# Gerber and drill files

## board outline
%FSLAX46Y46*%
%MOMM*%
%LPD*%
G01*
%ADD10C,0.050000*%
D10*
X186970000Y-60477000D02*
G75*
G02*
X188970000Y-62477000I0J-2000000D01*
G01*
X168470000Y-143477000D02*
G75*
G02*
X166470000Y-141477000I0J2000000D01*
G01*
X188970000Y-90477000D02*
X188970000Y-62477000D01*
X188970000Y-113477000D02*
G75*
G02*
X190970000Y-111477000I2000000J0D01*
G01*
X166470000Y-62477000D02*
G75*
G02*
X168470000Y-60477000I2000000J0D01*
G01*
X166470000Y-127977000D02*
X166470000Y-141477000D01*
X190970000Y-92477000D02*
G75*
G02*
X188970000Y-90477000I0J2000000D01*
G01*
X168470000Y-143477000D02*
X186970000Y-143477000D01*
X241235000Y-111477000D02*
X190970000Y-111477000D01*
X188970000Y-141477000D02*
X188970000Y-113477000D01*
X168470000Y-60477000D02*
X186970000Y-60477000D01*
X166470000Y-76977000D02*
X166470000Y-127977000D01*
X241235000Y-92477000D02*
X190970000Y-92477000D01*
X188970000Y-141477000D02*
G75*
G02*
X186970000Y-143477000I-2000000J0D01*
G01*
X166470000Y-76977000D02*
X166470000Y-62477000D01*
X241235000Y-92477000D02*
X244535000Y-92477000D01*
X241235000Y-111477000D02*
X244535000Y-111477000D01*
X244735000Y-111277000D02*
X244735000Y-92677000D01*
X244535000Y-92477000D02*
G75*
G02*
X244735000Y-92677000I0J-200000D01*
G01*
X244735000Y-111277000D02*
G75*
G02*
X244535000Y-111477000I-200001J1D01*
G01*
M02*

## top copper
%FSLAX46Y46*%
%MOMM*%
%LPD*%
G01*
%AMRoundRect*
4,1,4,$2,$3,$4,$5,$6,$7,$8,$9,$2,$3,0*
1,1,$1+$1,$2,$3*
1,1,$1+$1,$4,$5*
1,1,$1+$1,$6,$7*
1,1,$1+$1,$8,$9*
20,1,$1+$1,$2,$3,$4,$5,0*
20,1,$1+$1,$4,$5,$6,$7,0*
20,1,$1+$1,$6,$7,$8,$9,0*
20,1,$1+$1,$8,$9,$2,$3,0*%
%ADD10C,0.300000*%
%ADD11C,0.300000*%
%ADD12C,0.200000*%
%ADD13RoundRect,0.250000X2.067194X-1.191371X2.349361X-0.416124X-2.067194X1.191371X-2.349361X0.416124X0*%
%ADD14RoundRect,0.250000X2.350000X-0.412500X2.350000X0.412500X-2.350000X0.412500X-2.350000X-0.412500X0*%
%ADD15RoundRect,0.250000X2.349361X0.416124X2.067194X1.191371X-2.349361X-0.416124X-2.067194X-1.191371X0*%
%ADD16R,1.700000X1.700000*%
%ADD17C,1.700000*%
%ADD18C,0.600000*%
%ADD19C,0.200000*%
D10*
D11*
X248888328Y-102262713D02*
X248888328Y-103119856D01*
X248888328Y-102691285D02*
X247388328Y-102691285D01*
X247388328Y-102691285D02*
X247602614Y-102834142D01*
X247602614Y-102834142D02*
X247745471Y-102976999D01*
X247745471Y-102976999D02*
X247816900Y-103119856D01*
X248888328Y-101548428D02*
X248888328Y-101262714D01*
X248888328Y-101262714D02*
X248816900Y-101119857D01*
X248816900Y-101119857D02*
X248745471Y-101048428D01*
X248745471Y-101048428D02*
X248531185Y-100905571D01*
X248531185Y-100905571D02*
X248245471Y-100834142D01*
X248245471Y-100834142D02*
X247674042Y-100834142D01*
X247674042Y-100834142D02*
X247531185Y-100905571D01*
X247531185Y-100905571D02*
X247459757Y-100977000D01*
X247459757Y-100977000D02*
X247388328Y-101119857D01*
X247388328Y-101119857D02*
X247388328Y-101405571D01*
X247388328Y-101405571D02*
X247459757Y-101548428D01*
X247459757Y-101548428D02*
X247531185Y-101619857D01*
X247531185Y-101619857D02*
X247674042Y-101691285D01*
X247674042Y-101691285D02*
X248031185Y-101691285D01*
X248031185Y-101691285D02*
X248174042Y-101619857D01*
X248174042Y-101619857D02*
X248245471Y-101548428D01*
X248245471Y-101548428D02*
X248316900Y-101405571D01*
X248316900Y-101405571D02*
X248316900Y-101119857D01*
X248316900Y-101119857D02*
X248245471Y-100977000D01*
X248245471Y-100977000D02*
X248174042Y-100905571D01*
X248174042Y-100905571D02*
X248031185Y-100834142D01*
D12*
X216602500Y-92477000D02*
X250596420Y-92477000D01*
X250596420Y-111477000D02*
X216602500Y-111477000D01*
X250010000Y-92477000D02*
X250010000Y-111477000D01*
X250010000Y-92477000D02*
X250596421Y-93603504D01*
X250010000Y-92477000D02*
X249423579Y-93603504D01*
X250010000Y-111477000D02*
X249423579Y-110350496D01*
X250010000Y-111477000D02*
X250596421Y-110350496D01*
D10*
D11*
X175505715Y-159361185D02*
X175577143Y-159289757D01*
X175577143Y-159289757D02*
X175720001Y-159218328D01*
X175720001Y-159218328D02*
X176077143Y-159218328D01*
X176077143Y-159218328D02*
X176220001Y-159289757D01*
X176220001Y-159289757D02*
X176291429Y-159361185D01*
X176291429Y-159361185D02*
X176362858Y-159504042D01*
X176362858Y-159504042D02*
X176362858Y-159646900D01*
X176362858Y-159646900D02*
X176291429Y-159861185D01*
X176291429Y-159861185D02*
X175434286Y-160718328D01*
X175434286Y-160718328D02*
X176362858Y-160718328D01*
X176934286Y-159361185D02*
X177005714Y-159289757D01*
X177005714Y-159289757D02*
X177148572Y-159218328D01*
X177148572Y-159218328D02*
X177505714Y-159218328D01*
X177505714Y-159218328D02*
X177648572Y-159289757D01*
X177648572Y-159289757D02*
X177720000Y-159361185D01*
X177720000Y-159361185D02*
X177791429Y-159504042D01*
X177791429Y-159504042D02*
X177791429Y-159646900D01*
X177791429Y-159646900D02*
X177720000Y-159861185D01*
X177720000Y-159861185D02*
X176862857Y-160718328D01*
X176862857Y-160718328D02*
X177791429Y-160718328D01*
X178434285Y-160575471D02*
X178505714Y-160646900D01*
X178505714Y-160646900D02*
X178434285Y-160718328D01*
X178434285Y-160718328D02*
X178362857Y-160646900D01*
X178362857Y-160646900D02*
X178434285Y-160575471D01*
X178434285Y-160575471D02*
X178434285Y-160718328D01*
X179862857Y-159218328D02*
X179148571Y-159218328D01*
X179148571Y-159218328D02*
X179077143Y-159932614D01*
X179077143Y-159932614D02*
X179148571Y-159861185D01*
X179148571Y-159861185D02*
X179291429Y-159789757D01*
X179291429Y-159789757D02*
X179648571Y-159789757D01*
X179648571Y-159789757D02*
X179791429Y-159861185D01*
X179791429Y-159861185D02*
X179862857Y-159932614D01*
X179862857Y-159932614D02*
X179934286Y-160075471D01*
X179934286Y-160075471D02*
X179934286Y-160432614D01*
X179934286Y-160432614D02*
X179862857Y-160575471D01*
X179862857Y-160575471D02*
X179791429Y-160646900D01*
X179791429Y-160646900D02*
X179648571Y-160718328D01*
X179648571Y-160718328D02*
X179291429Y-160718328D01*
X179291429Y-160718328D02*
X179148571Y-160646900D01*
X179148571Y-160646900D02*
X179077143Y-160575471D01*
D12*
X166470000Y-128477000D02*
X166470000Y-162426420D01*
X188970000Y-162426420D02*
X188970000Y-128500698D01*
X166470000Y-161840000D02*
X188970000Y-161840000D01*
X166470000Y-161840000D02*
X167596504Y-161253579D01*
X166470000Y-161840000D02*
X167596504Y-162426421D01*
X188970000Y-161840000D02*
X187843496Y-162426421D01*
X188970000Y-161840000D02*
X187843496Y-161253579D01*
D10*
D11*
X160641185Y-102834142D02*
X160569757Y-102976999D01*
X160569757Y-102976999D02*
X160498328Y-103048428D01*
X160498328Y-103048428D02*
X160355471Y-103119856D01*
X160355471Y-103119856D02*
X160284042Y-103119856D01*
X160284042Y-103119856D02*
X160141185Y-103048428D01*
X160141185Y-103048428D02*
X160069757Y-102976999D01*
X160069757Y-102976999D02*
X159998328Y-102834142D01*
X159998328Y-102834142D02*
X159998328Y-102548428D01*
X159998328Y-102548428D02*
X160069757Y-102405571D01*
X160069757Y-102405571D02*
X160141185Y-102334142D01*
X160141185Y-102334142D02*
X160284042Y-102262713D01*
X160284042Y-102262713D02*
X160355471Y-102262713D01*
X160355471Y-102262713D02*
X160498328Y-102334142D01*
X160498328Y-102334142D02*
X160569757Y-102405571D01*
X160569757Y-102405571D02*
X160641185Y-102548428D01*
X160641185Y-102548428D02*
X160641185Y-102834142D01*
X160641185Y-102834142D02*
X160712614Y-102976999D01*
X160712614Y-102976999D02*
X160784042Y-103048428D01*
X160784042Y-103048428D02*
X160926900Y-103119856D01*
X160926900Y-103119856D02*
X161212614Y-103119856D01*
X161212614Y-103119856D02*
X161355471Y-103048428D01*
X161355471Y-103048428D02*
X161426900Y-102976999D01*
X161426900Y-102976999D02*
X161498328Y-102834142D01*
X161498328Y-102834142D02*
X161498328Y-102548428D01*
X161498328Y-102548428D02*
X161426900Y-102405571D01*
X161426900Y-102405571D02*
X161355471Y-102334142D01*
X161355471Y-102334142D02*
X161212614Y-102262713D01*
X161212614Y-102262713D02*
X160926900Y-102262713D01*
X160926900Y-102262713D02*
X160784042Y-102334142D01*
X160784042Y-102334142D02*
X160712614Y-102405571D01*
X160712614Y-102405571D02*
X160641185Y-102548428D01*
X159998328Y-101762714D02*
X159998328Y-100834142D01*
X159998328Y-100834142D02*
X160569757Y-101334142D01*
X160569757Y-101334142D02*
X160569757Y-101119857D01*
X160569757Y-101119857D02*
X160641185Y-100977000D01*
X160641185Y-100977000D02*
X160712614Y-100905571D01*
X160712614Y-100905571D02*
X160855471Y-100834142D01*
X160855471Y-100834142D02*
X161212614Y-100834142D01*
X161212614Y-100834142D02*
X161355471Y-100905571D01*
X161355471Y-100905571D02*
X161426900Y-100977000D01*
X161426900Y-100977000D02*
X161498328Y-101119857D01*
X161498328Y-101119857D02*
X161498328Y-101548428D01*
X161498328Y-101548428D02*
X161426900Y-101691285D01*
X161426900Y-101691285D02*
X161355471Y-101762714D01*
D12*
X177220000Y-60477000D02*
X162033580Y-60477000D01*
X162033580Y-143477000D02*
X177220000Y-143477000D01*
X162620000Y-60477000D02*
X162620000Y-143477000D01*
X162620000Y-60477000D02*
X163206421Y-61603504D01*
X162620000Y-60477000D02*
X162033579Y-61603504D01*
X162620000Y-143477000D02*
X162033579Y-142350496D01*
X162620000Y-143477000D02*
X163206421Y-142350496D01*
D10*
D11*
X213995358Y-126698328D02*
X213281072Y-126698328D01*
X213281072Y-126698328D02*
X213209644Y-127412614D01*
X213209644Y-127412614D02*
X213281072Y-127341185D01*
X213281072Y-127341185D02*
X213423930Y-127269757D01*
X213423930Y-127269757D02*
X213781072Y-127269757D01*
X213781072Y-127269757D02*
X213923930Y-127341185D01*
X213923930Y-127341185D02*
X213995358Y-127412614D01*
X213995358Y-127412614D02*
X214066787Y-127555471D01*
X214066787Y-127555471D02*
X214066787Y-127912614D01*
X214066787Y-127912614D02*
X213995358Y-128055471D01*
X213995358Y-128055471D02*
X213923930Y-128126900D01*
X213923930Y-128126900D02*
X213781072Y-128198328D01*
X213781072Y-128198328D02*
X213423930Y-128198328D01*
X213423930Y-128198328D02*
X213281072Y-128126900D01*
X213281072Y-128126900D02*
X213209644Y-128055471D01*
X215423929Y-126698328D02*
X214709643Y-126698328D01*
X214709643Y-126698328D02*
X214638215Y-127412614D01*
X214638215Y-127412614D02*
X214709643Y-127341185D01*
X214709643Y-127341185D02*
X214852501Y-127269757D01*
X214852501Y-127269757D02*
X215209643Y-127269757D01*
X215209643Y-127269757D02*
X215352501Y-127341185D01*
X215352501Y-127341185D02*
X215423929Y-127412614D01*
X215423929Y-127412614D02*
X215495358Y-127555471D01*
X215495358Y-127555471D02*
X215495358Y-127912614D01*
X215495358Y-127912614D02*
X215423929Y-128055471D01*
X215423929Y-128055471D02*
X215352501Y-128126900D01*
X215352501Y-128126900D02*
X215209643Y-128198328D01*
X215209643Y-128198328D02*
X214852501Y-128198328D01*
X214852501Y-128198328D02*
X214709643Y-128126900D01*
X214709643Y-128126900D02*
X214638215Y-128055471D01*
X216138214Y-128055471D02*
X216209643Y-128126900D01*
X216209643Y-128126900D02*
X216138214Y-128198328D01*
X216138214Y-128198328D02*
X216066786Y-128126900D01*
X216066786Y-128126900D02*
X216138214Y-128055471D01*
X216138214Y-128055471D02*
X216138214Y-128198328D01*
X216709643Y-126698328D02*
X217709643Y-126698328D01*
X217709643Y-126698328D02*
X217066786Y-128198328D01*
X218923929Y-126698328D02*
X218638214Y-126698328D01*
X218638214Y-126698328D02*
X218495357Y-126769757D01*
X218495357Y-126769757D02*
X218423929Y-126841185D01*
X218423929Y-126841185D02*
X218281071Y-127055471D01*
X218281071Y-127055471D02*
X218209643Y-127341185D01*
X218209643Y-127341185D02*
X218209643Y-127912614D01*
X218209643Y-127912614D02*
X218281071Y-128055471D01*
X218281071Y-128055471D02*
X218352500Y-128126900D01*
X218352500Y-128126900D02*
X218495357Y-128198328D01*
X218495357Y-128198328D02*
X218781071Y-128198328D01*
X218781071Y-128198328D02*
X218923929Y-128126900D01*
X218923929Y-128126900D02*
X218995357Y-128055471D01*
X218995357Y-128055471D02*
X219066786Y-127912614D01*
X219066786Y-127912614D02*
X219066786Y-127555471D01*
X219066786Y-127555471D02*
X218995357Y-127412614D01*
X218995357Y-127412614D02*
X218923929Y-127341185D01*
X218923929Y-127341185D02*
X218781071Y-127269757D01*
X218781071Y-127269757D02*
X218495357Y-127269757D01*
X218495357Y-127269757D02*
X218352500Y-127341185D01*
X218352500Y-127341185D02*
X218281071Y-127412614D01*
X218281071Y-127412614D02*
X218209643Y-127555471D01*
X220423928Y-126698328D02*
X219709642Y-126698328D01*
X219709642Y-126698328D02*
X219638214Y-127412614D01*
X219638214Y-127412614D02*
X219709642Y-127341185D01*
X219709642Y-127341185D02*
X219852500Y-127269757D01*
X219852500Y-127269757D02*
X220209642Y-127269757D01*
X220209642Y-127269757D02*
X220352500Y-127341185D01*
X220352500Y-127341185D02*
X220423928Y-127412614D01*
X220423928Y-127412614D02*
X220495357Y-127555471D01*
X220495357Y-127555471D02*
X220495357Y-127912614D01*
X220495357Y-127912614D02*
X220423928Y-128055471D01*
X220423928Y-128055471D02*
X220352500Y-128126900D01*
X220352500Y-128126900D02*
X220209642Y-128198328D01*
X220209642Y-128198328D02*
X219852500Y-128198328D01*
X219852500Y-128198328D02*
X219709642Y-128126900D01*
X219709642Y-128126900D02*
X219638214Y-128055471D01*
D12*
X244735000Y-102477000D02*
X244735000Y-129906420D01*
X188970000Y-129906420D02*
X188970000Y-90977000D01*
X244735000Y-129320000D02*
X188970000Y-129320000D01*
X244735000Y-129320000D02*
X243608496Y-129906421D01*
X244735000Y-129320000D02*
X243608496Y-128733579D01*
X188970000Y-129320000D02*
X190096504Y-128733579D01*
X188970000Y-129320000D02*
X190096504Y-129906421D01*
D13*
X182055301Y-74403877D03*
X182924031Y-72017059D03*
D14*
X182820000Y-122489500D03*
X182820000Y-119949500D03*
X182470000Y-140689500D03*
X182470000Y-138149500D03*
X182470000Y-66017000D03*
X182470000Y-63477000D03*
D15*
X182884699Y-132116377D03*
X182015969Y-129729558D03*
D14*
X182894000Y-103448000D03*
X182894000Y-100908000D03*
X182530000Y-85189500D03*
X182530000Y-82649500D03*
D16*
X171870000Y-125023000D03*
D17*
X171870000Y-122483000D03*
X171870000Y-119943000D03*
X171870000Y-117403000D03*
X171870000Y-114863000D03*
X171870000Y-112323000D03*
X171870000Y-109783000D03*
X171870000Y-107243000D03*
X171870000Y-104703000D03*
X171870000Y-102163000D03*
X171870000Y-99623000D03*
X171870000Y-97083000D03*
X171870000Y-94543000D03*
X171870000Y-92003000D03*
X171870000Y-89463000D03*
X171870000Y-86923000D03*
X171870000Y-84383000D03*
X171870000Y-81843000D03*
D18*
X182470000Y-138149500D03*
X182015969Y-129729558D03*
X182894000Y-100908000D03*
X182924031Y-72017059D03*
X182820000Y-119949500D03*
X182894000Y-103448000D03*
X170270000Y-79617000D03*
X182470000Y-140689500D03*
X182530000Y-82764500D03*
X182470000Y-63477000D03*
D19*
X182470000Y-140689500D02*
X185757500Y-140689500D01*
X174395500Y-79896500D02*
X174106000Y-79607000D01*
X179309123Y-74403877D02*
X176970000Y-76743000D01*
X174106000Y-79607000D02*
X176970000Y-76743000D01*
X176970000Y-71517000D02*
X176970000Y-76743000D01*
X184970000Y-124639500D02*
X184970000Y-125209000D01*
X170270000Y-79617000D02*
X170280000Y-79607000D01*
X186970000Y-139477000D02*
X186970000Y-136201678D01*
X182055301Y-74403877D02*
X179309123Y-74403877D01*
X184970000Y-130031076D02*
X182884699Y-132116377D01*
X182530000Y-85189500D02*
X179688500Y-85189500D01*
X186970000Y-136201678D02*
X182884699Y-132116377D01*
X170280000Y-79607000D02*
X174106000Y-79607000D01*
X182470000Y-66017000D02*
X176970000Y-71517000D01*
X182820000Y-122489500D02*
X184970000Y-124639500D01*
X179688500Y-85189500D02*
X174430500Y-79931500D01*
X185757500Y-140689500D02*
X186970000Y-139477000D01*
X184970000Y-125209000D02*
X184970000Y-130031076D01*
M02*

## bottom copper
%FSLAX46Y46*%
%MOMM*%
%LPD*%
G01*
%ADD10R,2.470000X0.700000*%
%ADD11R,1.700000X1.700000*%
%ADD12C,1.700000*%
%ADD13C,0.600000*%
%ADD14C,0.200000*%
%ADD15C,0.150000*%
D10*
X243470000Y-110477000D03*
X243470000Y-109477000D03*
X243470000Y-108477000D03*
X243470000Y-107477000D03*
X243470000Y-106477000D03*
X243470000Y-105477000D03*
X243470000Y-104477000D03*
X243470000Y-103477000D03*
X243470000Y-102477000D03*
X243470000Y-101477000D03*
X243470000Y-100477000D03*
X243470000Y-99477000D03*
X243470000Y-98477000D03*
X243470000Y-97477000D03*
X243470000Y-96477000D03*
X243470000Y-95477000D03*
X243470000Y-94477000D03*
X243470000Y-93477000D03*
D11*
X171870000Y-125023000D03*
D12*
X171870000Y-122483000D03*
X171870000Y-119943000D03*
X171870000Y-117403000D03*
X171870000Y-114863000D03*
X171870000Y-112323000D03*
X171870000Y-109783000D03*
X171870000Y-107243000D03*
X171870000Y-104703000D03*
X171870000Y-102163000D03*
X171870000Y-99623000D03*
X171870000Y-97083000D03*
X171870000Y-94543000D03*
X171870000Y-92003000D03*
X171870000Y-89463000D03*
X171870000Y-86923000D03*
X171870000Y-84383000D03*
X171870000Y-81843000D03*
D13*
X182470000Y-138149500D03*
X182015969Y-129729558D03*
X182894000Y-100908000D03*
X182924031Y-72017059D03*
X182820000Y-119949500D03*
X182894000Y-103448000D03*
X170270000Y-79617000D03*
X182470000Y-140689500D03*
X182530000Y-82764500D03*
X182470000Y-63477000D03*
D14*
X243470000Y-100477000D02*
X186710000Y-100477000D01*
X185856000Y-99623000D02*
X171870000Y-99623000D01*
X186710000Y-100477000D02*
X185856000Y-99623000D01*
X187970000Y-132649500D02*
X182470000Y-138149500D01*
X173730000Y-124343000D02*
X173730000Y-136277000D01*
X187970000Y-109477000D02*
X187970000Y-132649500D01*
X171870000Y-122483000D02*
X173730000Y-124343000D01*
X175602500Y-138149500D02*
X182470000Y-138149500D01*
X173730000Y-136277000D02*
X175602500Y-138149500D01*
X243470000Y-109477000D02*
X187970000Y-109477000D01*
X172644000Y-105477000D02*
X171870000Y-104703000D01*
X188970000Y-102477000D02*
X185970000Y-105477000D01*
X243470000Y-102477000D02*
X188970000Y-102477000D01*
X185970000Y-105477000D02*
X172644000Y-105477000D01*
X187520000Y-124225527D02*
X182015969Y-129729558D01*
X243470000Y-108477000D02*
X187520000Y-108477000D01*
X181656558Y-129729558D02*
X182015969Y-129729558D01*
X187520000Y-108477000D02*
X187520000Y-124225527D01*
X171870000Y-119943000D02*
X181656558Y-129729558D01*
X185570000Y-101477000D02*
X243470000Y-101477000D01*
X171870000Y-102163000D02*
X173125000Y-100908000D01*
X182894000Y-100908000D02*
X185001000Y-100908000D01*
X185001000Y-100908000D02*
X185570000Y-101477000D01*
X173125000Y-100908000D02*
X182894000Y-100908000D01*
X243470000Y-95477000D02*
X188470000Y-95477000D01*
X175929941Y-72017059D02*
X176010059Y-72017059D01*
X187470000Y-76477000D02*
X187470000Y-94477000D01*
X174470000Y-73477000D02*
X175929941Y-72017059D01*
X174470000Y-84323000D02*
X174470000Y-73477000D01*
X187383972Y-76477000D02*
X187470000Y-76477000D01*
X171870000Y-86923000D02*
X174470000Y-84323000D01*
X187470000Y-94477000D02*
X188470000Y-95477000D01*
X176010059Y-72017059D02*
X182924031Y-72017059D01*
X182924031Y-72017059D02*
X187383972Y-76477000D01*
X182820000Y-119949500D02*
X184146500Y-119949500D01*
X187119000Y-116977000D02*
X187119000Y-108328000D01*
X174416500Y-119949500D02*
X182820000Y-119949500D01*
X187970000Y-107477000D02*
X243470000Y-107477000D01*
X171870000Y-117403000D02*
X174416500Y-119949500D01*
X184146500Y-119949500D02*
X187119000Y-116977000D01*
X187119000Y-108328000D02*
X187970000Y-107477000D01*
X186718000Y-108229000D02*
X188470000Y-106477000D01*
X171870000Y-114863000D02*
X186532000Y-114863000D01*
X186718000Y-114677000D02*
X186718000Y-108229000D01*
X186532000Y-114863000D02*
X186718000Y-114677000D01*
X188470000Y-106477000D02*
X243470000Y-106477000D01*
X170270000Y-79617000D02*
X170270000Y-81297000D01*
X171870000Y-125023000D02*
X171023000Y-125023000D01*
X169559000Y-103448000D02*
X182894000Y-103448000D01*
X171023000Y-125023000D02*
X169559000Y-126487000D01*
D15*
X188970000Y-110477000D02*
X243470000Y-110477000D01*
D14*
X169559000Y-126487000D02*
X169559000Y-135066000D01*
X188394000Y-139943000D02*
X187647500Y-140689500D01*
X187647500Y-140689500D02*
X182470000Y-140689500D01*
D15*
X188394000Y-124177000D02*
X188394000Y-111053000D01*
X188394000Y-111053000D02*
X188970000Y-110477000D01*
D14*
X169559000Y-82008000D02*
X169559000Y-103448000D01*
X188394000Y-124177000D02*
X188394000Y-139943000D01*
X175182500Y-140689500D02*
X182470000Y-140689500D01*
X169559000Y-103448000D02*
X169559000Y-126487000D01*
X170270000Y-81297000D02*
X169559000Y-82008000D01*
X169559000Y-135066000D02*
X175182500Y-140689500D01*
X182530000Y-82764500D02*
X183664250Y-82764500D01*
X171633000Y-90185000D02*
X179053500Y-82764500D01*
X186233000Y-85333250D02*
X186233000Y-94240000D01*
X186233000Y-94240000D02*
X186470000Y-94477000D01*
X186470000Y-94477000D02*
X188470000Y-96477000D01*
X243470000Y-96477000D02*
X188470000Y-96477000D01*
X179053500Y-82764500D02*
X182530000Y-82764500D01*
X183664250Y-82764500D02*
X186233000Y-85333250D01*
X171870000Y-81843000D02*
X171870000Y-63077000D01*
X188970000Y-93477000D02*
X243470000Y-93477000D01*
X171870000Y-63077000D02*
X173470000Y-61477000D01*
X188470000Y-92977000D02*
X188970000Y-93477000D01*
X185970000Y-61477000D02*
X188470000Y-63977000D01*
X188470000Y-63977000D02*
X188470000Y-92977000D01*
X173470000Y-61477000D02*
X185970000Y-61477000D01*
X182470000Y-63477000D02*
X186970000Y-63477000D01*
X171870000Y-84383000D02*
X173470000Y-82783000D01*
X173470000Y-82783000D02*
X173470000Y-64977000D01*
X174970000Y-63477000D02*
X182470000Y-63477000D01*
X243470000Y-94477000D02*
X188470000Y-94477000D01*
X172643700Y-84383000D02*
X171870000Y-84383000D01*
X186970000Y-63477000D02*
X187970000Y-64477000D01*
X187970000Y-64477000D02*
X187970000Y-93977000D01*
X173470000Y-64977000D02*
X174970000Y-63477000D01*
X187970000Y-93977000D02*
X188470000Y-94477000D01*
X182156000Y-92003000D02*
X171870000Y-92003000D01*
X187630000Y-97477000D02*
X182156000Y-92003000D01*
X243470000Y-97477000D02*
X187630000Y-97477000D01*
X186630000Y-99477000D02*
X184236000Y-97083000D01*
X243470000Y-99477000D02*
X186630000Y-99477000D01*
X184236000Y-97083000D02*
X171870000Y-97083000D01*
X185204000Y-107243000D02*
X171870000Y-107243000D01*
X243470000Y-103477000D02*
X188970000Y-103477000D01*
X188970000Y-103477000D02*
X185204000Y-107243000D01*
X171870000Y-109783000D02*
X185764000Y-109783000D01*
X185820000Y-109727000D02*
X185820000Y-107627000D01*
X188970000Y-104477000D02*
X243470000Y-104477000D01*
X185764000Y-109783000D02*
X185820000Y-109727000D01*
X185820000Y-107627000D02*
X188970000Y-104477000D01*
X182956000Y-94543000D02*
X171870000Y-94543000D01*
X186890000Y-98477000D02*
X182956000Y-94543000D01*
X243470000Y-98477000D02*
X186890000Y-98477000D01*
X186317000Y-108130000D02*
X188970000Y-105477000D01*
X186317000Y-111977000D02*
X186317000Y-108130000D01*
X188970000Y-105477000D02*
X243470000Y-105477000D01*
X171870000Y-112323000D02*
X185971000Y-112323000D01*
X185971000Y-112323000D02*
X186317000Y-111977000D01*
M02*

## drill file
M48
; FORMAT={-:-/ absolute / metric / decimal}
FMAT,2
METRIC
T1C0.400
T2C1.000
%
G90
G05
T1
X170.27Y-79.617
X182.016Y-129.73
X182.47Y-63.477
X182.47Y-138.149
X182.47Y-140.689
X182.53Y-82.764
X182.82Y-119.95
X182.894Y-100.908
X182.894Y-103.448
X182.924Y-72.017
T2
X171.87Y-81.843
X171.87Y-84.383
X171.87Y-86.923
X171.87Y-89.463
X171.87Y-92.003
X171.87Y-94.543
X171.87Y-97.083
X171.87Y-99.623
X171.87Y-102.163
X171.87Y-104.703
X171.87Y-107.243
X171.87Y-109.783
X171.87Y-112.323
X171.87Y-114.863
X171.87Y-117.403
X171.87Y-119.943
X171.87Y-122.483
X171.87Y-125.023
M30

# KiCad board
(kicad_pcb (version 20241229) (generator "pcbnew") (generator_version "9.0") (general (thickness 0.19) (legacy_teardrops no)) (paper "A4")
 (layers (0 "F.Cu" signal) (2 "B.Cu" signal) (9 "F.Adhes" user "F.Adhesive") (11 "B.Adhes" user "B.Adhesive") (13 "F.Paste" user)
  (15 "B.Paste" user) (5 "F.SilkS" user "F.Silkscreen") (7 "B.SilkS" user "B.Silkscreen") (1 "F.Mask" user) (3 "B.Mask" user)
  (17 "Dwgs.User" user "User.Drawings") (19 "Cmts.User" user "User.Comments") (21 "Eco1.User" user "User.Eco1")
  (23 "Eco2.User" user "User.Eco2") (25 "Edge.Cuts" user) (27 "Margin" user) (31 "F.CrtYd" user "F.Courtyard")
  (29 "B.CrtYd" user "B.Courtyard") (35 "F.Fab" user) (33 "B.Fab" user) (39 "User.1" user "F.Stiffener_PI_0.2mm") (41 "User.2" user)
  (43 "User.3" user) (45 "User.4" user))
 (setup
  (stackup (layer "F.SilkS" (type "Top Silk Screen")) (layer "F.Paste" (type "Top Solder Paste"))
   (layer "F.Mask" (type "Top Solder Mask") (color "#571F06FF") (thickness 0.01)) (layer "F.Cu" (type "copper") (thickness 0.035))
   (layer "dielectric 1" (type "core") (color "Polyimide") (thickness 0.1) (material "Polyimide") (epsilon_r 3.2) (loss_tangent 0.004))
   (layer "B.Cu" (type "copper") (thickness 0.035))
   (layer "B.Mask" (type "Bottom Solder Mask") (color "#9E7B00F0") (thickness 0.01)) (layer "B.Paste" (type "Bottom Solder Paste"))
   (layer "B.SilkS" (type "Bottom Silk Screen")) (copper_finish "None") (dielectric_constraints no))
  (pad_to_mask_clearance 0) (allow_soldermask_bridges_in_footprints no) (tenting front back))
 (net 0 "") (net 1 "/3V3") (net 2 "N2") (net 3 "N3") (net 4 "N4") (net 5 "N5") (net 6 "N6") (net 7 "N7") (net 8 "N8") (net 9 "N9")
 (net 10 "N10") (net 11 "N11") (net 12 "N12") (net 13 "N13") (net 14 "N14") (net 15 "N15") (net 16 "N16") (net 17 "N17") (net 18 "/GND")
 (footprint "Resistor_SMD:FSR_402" (layer "F.Cu") (at 182.47 73.2645 70)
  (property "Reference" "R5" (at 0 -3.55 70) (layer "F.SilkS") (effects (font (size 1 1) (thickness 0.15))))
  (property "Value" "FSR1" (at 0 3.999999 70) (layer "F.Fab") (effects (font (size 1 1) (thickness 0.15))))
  (pad "1" smd roundrect (at -1.2125 0 70) (size 1.325 5.2) (layers "F.Cu" "F.Mask" "F.Paste") (roundrect_rratio 0.188679) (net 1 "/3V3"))
  (pad "2" smd roundrect (at 1.327499 0 70) (size 1.325 5.2) (layers "F.Cu" "F.Mask" "F.Paste") (roundrect_rratio 0.188679) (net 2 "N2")))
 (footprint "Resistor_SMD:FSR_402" (layer "F.Cu") (at 182.82 121.277 90)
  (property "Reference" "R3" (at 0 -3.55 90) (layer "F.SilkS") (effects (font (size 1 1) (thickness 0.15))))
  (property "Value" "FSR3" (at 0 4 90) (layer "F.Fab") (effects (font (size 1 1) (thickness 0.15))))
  (pad "1" smd roundrect (at -1.2125 0 90) (size 1.325 5.2) (layers "F.Cu" "F.Mask" "F.Paste") (roundrect_rratio 0.188679) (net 1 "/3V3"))
  (pad "2" smd roundrect (at 1.3275 0 90) (size 1.325 5.2) (layers "F.Cu" "F.Mask" "F.Paste") (roundrect_rratio 0.188679) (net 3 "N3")))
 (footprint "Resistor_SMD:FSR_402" (layer "F.Cu") (at 182.47 139.477 90)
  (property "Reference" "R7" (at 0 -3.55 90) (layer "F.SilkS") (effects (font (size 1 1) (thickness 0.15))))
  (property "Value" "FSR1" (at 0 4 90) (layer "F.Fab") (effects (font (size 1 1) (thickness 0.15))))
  (pad "1" smd roundrect (at -1.2125 0 90) (size 1.325 5.2) (layers "F.Cu" "F.Mask" "F.Paste") (roundrect_rratio 0.188679) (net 1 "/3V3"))
  (pad "2" smd roundrect (at 1.3275 0 90) (size 1.325 5.2) (layers "F.Cu" "F.Mask" "F.Paste") (roundrect_rratio 0.188679) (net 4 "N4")))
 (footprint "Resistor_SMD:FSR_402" (layer "F.Cu") (at 182.47 64.8045 90)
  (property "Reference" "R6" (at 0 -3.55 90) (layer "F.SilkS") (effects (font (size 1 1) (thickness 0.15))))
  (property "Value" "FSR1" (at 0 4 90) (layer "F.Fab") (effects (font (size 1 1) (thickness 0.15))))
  (pad "1" smd roundrect (at -1.2125 0 90) (size 1.325 5.2) (layers "F.Cu" "F.Mask" "F.Paste") (roundrect_rratio 0.188679) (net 1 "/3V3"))
  (pad "2" smd roundrect (at 1.3275 0 90) (size 1.325 5.2) (layers "F.Cu" "F.Mask" "F.Paste") (roundrect_rratio 0.188679) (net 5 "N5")))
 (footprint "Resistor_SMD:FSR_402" (layer "F.Cu") (at 182.47 130.977 110)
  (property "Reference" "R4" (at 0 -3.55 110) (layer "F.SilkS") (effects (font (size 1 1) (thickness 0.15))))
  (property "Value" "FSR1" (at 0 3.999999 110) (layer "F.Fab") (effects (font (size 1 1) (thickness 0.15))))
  (pad "1" smd roundrect (at -1.2125 0 110) (size 1.325 5.2) (layers "F.Cu" "F.Mask" "F.Paste") (roundrect_rratio 0.188679) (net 1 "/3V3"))
  (pad "2" smd roundrect (at 1.3275 0.000001 110) (size 1.325 5.2) (layers "F.Cu" "F.Mask" "F.Paste") (roundrect_rratio 0.188679)
   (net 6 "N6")))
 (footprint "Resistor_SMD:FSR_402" (layer "F.Cu") (at 182.894 102.2355 90)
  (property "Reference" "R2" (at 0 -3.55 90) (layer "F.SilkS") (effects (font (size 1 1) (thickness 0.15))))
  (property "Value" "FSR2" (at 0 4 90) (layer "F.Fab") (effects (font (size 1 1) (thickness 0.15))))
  (pad "1" smd roundrect (at -1.2125 0 90) (size 1.325 5.2) (layers "F.Cu" "F.Mask" "F.Paste") (roundrect_rratio 0.188679) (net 1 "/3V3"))
  (pad "2" smd roundrect (at 1.3275 0 90) (size 1.325 5.2) (layers "F.Cu" "F.Mask" "F.Paste") (roundrect_rratio 0.188679) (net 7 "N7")))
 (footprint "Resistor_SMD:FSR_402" (layer "F.Cu") (at 182.53 83.977 90)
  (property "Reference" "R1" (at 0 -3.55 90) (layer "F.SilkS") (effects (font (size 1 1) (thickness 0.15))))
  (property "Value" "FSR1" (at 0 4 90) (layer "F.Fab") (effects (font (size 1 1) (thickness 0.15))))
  (pad "1" smd roundrect (at -1.2125 0 90) (size 1.325 5.2) (layers "F.Cu" "F.Mask" "F.Paste") (roundrect_rratio 0.188679) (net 1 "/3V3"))
  (pad "2" smd roundrect (at 1.3275 0 90) (size 1.325 5.2) (layers "F.Cu" "F.Mask" "F.Paste") (roundrect_rratio 0.188679) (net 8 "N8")))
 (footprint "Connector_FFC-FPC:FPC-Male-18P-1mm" (layer "B.Cu") (at 243.43 102.387 90)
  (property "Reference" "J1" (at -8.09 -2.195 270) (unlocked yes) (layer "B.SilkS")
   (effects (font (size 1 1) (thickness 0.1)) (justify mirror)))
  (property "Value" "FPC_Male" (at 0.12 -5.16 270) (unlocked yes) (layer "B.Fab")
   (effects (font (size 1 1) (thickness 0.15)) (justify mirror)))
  (fp_line (start 9.91 -2.195) (end 9.91 1.105) (stroke (width 0.05) (type default)) (layer "Edge.Cuts"))
  (fp_line (start -9.09 -2.195) (end -9.09 1.105) (stroke (width 0.05) (type default)) (layer "Edge.Cuts"))
  (fp_line (start -8.89 1.305) (end 9.71 1.305) (stroke (width 0.05) (type default)) (layer "Edge.Cuts"))
  (fp_arc (start 9.91 1.105) (mid 9.851421 1.246421) (end 9.71 1.305) (stroke (width 0.05) (type default)) (layer "Edge.Cuts"))
  (fp_arc (start -8.89 1.305) (mid -9.031421 1.246421) (end -9.09 1.105) (stroke (width 0.05) (type default)) (layer "Edge.Cuts"))
  (pad "1" smd rect (at -8.09 0.04) (size 2.47 0.7) (layers "B.Cu" "B.Mask" "B.Paste") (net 1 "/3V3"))
  (pad "2" smd rect (at -7.09 0.04) (size 2.47 0.7) (layers "B.Cu" "B.Mask" "B.Paste") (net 4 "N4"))
  (pad "3" smd rect (at -6.09 0.04) (size 2.47 0.7) (layers "B.Cu" "B.Mask" "B.Paste") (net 6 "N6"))
  (pad "4" smd rect (at -5.09 0.04) (size 2.47 0.7) (layers "B.Cu" "B.Mask" "B.Paste") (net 3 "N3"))
  (pad "5" smd rect (at -4.09 0.04) (size 2.47 0.7) (layers "B.Cu" "B.Mask" "B.Paste") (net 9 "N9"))
  (pad "6" smd rect (at -3.09 0.04) (size 2.47 0.7) (layers "B.Cu" "B.Mask" "B.Paste") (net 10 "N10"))
  (pad "7" smd rect (at -2.09 0.04) (size 2.47 0.7) (layers "B.Cu" "B.Mask" "B.Paste") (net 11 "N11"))
  (pad "8" smd rect (at -1.09 0.04) (size 2.47 0.7) (layers "B.Cu" "B.Mask" "B.Paste") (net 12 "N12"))
  (pad "9" smd rect (at -0.09 0.04) (size 2.47 0.7) (layers "B.Cu" "B.Mask" "B.Paste") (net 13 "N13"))
  (pad "10" smd rect (at 0.91 0.04) (size 2.47 0.7) (layers "B.Cu" "B.Mask" "B.Paste") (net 7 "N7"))
  (pad "11" smd rect (at 1.91 0.04) (size 2.47 0.7) (layers "B.Cu" "B.Mask" "B.Paste") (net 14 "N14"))
  (pad "12" smd rect (at 2.91 0.04) (size 2.47 0.7) (layers "B.Cu" "B.Mask" "B.Paste") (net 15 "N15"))
  (pad "13" smd rect (at 3.91 0.04) (size 2.47 0.7) (layers "B.Cu" "B.Mask" "B.Paste") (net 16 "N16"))
  (pad "14" smd rect (at 4.91 0.04) (size 2.47 0.7) (layers "B.Cu" "B.Mask" "B.Paste") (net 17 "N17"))
  (pad "15" smd rect (at 5.91 0.04) (size 2.47 0.7) (layers "B.Cu" "B.Mask" "B.Paste") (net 8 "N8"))
  (pad "16" smd rect (at 6.91 0.04) (size 2.47 0.7) (layers "B.Cu" "B.Mask" "B.Paste") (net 2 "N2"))
  (pad "17" smd rect (at 7.91 0.04) (size 2.47 0.7) (layers "B.Cu" "B.Mask" "B.Paste") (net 5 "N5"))
  (pad "18" smd rect (at 8.91 0.04) (size 2.47 0.7) (layers "B.Cu" "B.Mask" "B.Paste") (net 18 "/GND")))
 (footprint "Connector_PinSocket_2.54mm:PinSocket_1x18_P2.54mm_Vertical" (layer "B.Cu") (at 171.87 125.023)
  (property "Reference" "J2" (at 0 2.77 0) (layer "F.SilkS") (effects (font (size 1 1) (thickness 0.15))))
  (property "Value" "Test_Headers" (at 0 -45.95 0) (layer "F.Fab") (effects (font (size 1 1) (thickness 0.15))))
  (pad "1" thru_hole rect (at 0 0) (size 1.7 1.7) (drill 1) (layers "*.Cu" "*.Mask") (remove_unused_layers no) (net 1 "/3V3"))
  (pad "2" thru_hole circle (at 0 -2.54) (size 1.7 1.7) (drill 1) (layers "*.Cu" "*.Mask") (remove_unused_layers no) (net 4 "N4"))
  (pad "3" thru_hole circle (at 0 -5.08) (size 1.7 1.7) (drill 1) (layers "*.Cu" "*.Mask") (remove_unused_layers no) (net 6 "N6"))
  (pad "4" thru_hole circle (at 0 -7.62) (size 1.7 1.7) (drill 1) (layers "*.Cu" "*.Mask") (remove_unused_layers no) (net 3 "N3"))
  (pad "5" thru_hole circle (at 0 -10.16) (size 1.7 1.7) (drill 1) (layers "*.Cu" "*.Mask") (remove_unused_layers no) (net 9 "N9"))
  (pad "6" thru_hole circle (at 0 -12.7) (size 1.7 1.7) (drill 1) (layers "*.Cu" "*.Mask") (remove_unused_layers no) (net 10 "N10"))
  (pad "7" thru_hole circle (at 0 -15.24) (size 1.7 1.7) (drill 1) (layers "*.Cu" "*.Mask") (remove_unused_layers no) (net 11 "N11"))
  (pad "8" thru_hole circle (at 0 -17.78) (size 1.7 1.7) (drill 1) (layers "*.Cu" "*.Mask") (remove_unused_layers no) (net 12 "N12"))
  (pad "9" thru_hole circle (at 0 -20.32) (size 1.7 1.7) (drill 1) (layers "*.Cu" "*.Mask") (remove_unused_layers no) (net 13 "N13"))
  (pad "10" thru_hole circle (at 0 -22.86) (size 1.7 1.7) (drill 1) (layers "*.Cu" "*.Mask") (remove_unused_layers no) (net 7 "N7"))
  (pad "11" thru_hole circle (at 0 -25.4) (size 1.7 1.7) (drill 1) (layers "*.Cu" "*.Mask") (remove_unused_layers no) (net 14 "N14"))
  (pad "12" thru_hole circle (at 0 -27.94) (size 1.7 1.7) (drill 1) (layers "*.Cu" "*.Mask") (remove_unused_layers no) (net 15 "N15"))
  (pad "13" thru_hole circle (at 0 -30.48) (size 1.7 1.7) (drill 1) (layers "*.Cu" "*.Mask") (remove_unused_layers no) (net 16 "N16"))
  (pad "14" thru_hole circle (at 0 -33.02) (size 1.7 1.7) (drill 1) (layers "*.Cu" "*.Mask") (remove_unused_layers no) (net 17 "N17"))
  (pad "15" thru_hole circle (at 0 -35.56) (size 1.7 1.7) (drill 1) (layers "*.Cu" "*.Mask") (remove_unused_layers no) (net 8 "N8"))
  (pad "16" thru_hole circle (at 0 -38.1) (size 1.7 1.7) (drill 1) (layers "*.Cu" "*.Mask") (remove_unused_layers no) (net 2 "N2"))
  (pad "17" thru_hole circle (at 0 -40.64) (size 1.7 1.7) (drill 1) (layers "*.Cu" "*.Mask") (remove_unused_layers no) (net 5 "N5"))
  (pad "18" thru_hole circle (at 0 -43.18) (size 1.7 1.7) (drill 1) (layers "*.Cu" "*.Mask") (remove_unused_layers no) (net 18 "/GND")))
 (gr_arc (start 186.97 60.477) (mid 188.384214 61.062786) (end 188.97 62.477) (stroke (width 0.05) (type default)) (layer "Edge.Cuts"))
 (gr_arc (start 168.47 143.477) (mid 167.055786 142.891214) (end 166.47 141.477) (stroke (width 0.05) (type default)) (layer "Edge.Cuts"))
 (gr_line (start 188.97 90.477) (end 188.97 62.477) (stroke (width 0.05) (type default)) (layer "Edge.Cuts"))
 (gr_arc (start 188.97 113.477) (mid 189.555786 112.062786) (end 190.97 111.477) (stroke (width 0.05) (type default)) (layer "Edge.Cuts"))
 (gr_arc (start 166.47 62.477) (mid 167.055786 61.062786) (end 168.47 60.477) (stroke (width 0.05) (type default)) (layer "Edge.Cuts"))
 (gr_line (start 166.47 127.977) (end 166.47 141.477) (stroke (width 0.05) (type default)) (layer "Edge.Cuts"))
 (gr_arc (start 190.97 92.477) (mid 189.555786 91.891214) (end 188.97 90.477) (stroke (width 0.05) (type default)) (layer "Edge.Cuts"))
 (gr_line (start 168.47 143.477) (end 186.97 143.477) (stroke (width 0.05) (type default)) (layer "Edge.Cuts"))
 (gr_line (start 241.235 111.477) (end 190.97 111.477) (stroke (width 0.05) (type default)) (layer "Edge.Cuts"))
 (gr_line (start 188.97 141.477) (end 188.97 113.477) (stroke (width 0.05) (type default)) (layer "Edge.Cuts"))
 (gr_line (start 168.47 60.477) (end 186.97 60.477) (stroke (width 0.05) (type default)) (layer "Edge.Cuts"))
 (gr_line (start 166.47 76.977) (end 166.47 127.977) (stroke (width 0.05) (type default)) (layer "Edge.Cuts"))
 (gr_line (start 241.235 92.477) (end 190.97 92.477) (stroke (width 0.05) (type default)) (layer "Edge.Cuts"))
 (gr_arc (start 188.97 141.477) (mid 188.384214 142.891214) (end 186.97 143.477) (stroke (width 0.05) (type default)) (layer "Edge.Cuts"))
 (gr_line (start 166.47 76.977) (end 166.47 62.477) (stroke (width 0.05) (type default)) (layer "Edge.Cuts"))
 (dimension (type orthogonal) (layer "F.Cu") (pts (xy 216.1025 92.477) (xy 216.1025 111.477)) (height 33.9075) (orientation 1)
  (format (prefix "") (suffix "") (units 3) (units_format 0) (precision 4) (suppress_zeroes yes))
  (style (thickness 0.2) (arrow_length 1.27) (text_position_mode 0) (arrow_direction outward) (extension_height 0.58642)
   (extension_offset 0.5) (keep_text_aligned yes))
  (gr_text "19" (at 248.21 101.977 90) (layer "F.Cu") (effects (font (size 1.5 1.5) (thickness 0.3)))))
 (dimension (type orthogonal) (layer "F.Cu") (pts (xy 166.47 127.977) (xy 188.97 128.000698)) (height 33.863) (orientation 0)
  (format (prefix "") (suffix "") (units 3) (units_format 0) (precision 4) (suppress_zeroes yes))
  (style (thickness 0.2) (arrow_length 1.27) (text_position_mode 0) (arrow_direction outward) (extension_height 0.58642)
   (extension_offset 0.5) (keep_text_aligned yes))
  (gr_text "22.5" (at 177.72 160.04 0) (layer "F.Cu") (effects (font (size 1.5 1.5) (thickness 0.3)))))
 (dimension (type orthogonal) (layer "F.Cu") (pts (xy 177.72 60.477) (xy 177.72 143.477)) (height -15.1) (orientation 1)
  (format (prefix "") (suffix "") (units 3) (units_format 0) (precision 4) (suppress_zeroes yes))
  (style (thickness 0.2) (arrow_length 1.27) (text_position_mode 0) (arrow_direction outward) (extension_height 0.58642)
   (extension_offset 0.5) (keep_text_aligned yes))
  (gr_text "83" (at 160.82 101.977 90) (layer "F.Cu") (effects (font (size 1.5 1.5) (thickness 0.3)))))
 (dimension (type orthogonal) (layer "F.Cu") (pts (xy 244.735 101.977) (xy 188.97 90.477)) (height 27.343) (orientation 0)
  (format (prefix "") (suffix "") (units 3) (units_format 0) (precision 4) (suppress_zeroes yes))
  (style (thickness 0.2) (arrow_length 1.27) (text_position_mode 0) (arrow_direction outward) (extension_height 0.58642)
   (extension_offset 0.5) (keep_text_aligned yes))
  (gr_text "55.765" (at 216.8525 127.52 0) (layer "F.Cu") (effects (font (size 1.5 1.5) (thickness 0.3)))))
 (segment (start 243.47 100.477) (end 186.71 100.477) (width 0.2) (layer "B.Cu") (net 14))
 (segment (start 185.856 99.623) (end 171.87 99.623) (width 0.2) (layer "B.Cu") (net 14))
 (segment (start 186.71 100.477) (end 185.856 99.623) (width 0.2) (layer "B.Cu") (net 14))
 (via (at 182.47 138.1495) (size 0.6) (drill 0.4) (layers "F.Cu" "B.Cu") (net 4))
 (segment (start 187.97 132.6495) (end 182.47 138.1495) (width 0.2) (layer "B.Cu") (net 4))
 (segment (start 173.73 124.343) (end 173.73 136.277) (width 0.2) (layer "B.Cu") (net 4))
 (segment (start 187.97 109.477) (end 187.97 132.6495) (width 0.2) (layer "B.Cu") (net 4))
 (segment (start 171.87 122.483) (end 173.73 124.343) (width 0.2) (layer "B.Cu") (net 4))
 (segment (start 175.6025 138.1495) (end 182.47 138.1495) (width 0.2) (layer "B.Cu") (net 4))
 (segment (start 173.73 136.277) (end 175.6025 138.1495) (width 0.2) (layer "B.Cu") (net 4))
 (segment (start 243.47 109.477) (end 187.97 109.477) (width 0.2) (layer "B.Cu") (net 4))
 (segment (start 172.644 105.477) (end 171.87 104.703) (width 0.2) (layer "B.Cu") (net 13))
 (segment (start 188.97 102.477) (end 185.97 105.477) (width 0.2) (layer "B.Cu") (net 13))
 (segment (start 243.47 102.477) (end 188.97 102.477) (width 0.2) (layer "B.Cu") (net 13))
 (segment (start 185.97 105.477) (end 172.644 105.477) (width 0.2) (layer "B.Cu") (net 13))
 (via (at 182.015969 129.729558) (size 0.6) (drill 0.4) (layers "F.Cu" "B.Cu") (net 6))
 (segment (start 187.52 124.225527) (end 182.015969 129.729558) (width 0.2) (layer "B.Cu") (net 6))
 (segment (start 243.47 108.477) (end 187.52 108.477) (width 0.2) (layer "B.Cu") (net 6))
 (segment (start 181.656558 129.729558) (end 182.015969 129.729558) (width 0.2) (layer "B.Cu") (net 6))
 (segment (start 187.52 108.477) (end 187.52 124.225527) (width 0.2) (layer "B.Cu") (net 6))
 (segment (start 171.87 119.943) (end 181.656558 129.729558) (width 0.2) (layer "B.Cu") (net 6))
 (via (at 182.894 100.908) (size 0.6) (drill 0.4) (layers "F.Cu" "B.Cu") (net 7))
 (segment (start 185.57 101.477) (end 243.47 101.477) (width 0.2) (layer "B.Cu") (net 7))
 (segment (start 171.87 102.163) (end 173.125 100.908) (width 0.2) (layer "B.Cu") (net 7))
 (segment (start 182.894 100.908) (end 185.001 100.908) (width 0.2) (layer "B.Cu") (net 7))
 (segment (start 185.001 100.908) (end 185.57 101.477) (width 0.2) (layer "B.Cu") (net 7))
 (segment (start 173.125 100.908) (end 182.894 100.908) (width 0.2) (layer "B.Cu") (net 7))
 (via (at 182.924031 72.017059) (size 0.6) (drill 0.4) (layers "F.Cu" "B.Cu") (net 2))
 (segment (start 243.47 95.477) (end 188.47 95.477) (width 0.2) (layer "B.Cu") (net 2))
 (segment (start 175.929941 72.017059) (end 176.010059 72.017059) (width 0.2) (layer "B.Cu") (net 2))
 (segment (start 187.47 76.477) (end 187.47 94.477) (width 0.2) (layer "B.Cu") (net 2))
 (segment (start 174.47 73.477) (end 175.929941 72.017059) (width 0.2) (layer "B.Cu") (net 2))
 (segment (start 174.47 84.323) (end 174.47 73.477) (width 0.2) (layer "B.Cu") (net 2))
 (segment (start 187.383972 76.477) (end 187.47 76.477) (width 0.2) (layer "B.Cu") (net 2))
 (segment (start 171.87 86.923) (end 174.47 84.323) (width 0.2) (layer "B.Cu") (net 2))
 (segment (start 187.47 94.477) (end 188.47 95.477) (width 0.2) (layer "B.Cu") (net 2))
 (segment (start 176.010059 72.017059) (end 182.924031 72.017059) (width 0.2) (layer "B.Cu") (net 2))
 (segment (start 182.924031 72.017059) (end 187.383972 76.477) (width 0.2) (layer "B.Cu") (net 2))
 (via (at 182.82 119.9495) (size 0.6) (drill 0.4) (layers "F.Cu" "B.Cu") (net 3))
 (segment (start 182.82 119.9495) (end 184.1465 119.9495) (width 0.2) (layer "B.Cu") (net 3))
 (segment (start 187.119 116.977) (end 187.119 108.328) (width 0.2) (layer "B.Cu") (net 3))
 (segment (start 174.4165 119.9495) (end 182.82 119.9495) (width 0.2) (layer "B.Cu") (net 3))
 (segment (start 187.97 107.477) (end 243.47 107.477) (width 0.2) (layer "B.Cu") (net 3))
 (segment (start 171.87 117.403) (end 174.4165 119.9495) (width 0.2) (layer "B.Cu") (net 3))
 (segment (start 184.1465 119.9495) (end 187.119 116.977) (width 0.2) (layer "B.Cu") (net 3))
 (segment (start 187.119 108.328) (end 187.97 107.477) (width 0.2) (layer "B.Cu") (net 3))
 (segment (start 186.718 108.229) (end 188.47 106.477) (width 0.2) (layer "B.Cu") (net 9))
 (segment (start 171.87 114.863) (end 186.532 114.863) (width 0.2) (layer "B.Cu") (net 9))
 (segment (start 186.718 114.677) (end 186.718 108.229) (width 0.2) (layer "B.Cu") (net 9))
 (segment (start 186.532 114.863) (end 186.718 114.677) (width 0.2) (layer "B.Cu") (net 9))
 (segment (start 188.47 106.477) (end 243.47 106.477) (width 0.2) (layer "B.Cu") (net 9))
 (segment (start 182.47 140.6895) (end 185.7575 140.6895) (width 0.2) (layer "F.Cu") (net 1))
 (segment (start 174.3955 79.8965) (end 174.106 79.607) (width 0.2) (layer "F.Cu") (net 1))
 (segment (start 179.309123 74.403877) (end 176.97 76.743) (width 0.2) (layer "F.Cu") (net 1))
 (segment (start 174.106 79.607) (end 176.97 76.743) (width 0.2) (layer "F.Cu") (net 1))
 (segment (start 176.97 71.517) (end 176.97 76.743) (width 0.2) (layer "F.Cu") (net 1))
 (segment (start 184.97 124.6395) (end 184.97 125.209) (width 0.2) (layer "F.Cu") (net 1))
 (segment (start 170.27 79.617) (end 170.28 79.607) (width 0.2) (layer "F.Cu") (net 1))
 (segment (start 186.97 139.477) (end 186.97 136.201678) (width 0.2) (layer "F.Cu") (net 1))
 (segment (start 182.055301 74.403877) (end 179.309123 74.403877) (width 0.2) (layer "F.Cu") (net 1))
 (segment (start 184.97 130.031076) (end 182.884699 132.116377) (width 0.2) (layer "F.Cu") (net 1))
 (segment (start 182.53 85.1895) (end 179.6885 85.1895) (width 0.2) (layer "F.Cu") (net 1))
 (segment (start 186.97 136.201678) (end 182.884699 132.116377) (width 0.2) (layer "F.Cu") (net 1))
 (segment (start 170.28 79.607) (end 174.106 79.607) (width 0.2) (layer "F.Cu") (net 1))
 (segment (start 182.47 66.017) (end 176.97 71.517) (width 0.2) (layer "F.Cu") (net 1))
 (segment (start 182.82 122.4895) (end 184.97 124.6395) (width 0.2) (layer "F.Cu") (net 1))
 (segment (start 179.6885 85.1895) (end 174.4305 79.9315) (width 0.2) (layer "F.Cu") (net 1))
 (segment (start 185.7575 140.6895) (end 186.97 139.477) (width 0.2) (layer "F.Cu") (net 1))
 (segment (start 184.97 125.209) (end 184.97 130.031076) (width 0.2) (layer "F.Cu") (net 1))
 (via (at 182.894 103.448) (size 0.6) (drill 0.4) (layers "F.Cu" "B.Cu") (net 1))
 (via (at 170.27 79.617) (size 0.6) (drill 0.4) (layers "F.Cu" "B.Cu") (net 1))
 (via (at 182.47 140.6895) (size 0.6) (drill 0.4) (layers "F.Cu" "B.Cu") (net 1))
 (segment (start 170.27 79.617) (end 170.27 81.297) (width 0.2) (layer "B.Cu") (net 1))
 (segment (start 171.87 125.023) (end 171.023 125.023) (width 0.2) (layer "B.Cu") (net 1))
 (segment (start 169.559 103.448) (end 182.894 103.448) (width 0.2) (layer "B.Cu") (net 1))
 (segment (start 171.023 125.023) (end 169.559 126.487) (width 0.2) (layer "B.Cu") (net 1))
 (segment (start 188.97 110.477) (end 243.47 110.477) (width 0.15) (layer "B.Cu") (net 1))
 (segment (start 169.559 126.487) (end 169.559 135.066) (width 0.2) (layer "B.Cu") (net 1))
 (segment (start 188.394 139.943) (end 187.6475 140.6895) (width 0.2) (layer "B.Cu") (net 1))
 (segment (start 187.6475 140.6895) (end 182.47 140.6895) (width 0.2) (layer "B.Cu") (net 1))
 (segment (start 188.394 124.177) (end 188.394 111.053) (width 0.15) (layer "B.Cu") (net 1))
 (segment (start 188.394 111.053) (end 188.97 110.477) (width 0.15) (layer "B.Cu") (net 1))
 (segment (start 169.559 82.008) (end 169.559 103.448) (width 0.2) (layer "B.Cu") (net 1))
 (segment (start 188.394 124.177) (end 188.394 139.943) (width 0.2) (layer "B.Cu") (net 1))
 (segment (start 175.1825 140.6895) (end 182.47 140.6895) (width 0.2) (layer "B.Cu") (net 1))
 (segment (start 169.559 103.448) (end 169.559 126.487) (width 0.2) (layer "B.Cu") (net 1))
 (segment (start 170.27 81.297) (end 169.559 82.008) (width 0.2) (layer "B.Cu") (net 1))
 (segment (start 169.559 135.066) (end 175.1825 140.6895) (width 0.2) (layer "B.Cu") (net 1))
 (via (at 182.53 82.7645) (size 0.6) (drill 0.4) (layers "F.Cu" "B.Cu") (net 8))
 (segment (start 182.53 82.7645) (end 183.66425 82.7645) (width 0.2) (layer "B.Cu") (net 8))
 (segment (start 171.633 90.185) (end 179.0535 82.7645) (width 0.2) (layer "B.Cu") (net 8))
 (segment (start 186.233 85.33325) (end 186.233 94.24) (width 0.2) (layer "B.Cu") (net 8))
 (segment (start 186.233 94.24) (end 186.47 94.477) (width 0.2) (layer "B.Cu") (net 8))
 (segment (start 186.47 94.477) (end 188.47 96.477) (width 0.2) (layer "B.Cu") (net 8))
 (segment (start 243.47 96.477) (end 188.47 96.477) (width 0.2) (layer "B.Cu") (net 8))
 (segment (start 179.0535 82.7645) (end 182.53 82.7645) (width 0.2) (layer "B.Cu") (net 8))
 (segment (start 183.66425 82.7645) (end 186.233 85.33325) (width 0.2) (layer "B.Cu") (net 8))
 (segment (start 171.87 81.843) (end 171.87 63.077) (width 0.2) (layer "B.Cu") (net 18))
 (segment (start 188.97 93.477) (end 243.47 93.477) (width 0.2) (layer "B.Cu") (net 18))
 (segment (start 171.87 63.077) (end 173.47 61.477) (width 0.2) (layer "B.Cu") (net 18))
 (segment (start 188.47 92.977) (end 188.97 93.477) (width 0.2) (layer "B.Cu") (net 18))
 (segment (start 185.97 61.477) (end 188.47 63.977) (width 0.2) (layer "B.Cu") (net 18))
 (segment (start 188.47 63.977) (end 188.47 92.977) (width 0.2) (layer "B.Cu") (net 18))
 (segment (start 173.47 61.477) (end 185.97 61.477) (width 0.2) (layer "B.Cu") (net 18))
 (via (at 182.47 63.477) (size 0.6) (drill 0.4) (layers "F.Cu" "B.Cu") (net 5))
 (segment (start 182.47 63.477) (end 186.97 63.477) (width 0.2) (layer "B.Cu") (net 5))
 (segment (start 171.87 84.383) (end 173.47 82.783) (width 0.2) (layer "B.Cu") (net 5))
 (segment (start 173.47 82.783) (end 173.47 64.977) (width 0.2) (layer "B.Cu") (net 5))
 (segment (start 174.97 63.477) (end 182.47 63.477) (width 0.2) (layer "B.Cu") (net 5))
 (segment (start 243.47 94.477) (end 188.47 94.477) (width 0.2) (layer "B.Cu") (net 5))
 (segment (start 172.6437 84.383) (end 171.87 84.383) (width 0.2) (layer "B.Cu") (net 5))
 (segment (start 186.97 63.477) (end 187.97 64.477) (width 0.2) (layer "B.Cu") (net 5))
 (segment (start 187.97 64.477) (end 187.97 93.977) (width 0.2) (layer "B.Cu") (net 5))
 (segment (start 173.47 64.977) (end 174.97 63.477) (width 0.2) (layer "B.Cu") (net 5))
 (segment (start 187.97 93.977) (end 188.47 94.477) (width 0.2) (layer "B.Cu") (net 5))
 (segment (start 182.156 92.003) (end 171.87 92.003) (width 0.2) (layer "B.Cu") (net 17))
 (segment (start 187.63 97.477) (end 182.156 92.003) (width 0.2) (layer "B.Cu") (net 17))
 (segment (start 243.47 97.477) (end 187.63 97.477) (width 0.2) (layer "B.Cu") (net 17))
 (segment (start 186.63 99.477) (end 184.236 97.083) (width 0.2) (layer "B.Cu") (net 15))
 (segment (start 243.47 99.477) (end 186.63 99.477) (width 0.2) (layer "B.Cu") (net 15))
 (segment (start 184.236 97.083) (end 171.87 97.083) (width 0.2) (layer "B.Cu") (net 15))
 (segment (start 185.204 107.243) (end 171.87 107.243) (width 0.2) (layer "B.Cu") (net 12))
 (segment (start 243.47 103.477) (end 188.97 103.477) (width 0.2) (layer "B.Cu") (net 12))
 (segment (start 188.97 103.477) (end 185.204 107.243) (width 0.2) (layer "B.Cu") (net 12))
 (segment (start 171.87 109.783) (end 185.764 109.783) (width 0.2) (layer "B.Cu") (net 11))
 (segment (start 185.82 109.727) (end 185.82 107.627) (width 0.2) (layer "B.Cu") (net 11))
 (segment (start 188.97 104.477) (end 243.47 104.477) (width 0.2) (layer "B.Cu") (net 11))
 (segment (start 185.764 109.783) (end 185.82 109.727) (width 0.2) (layer "B.Cu") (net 11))
 (segment (start 185.82 107.627) (end 188.97 104.477) (width 0.2) (layer "B.Cu") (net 11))
 (segment (start 182.956 94.543) (end 171.87 94.543) (width 0.2) (layer "B.Cu") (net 16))
 (segment (start 186.89 98.477) (end 182.956 94.543) (width 0.2) (layer "B.Cu") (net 16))
 (segment (start 243.47 98.477) (end 186.89 98.477) (width 0.2) (layer "B.Cu") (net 16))
 (segment (start 186.317 108.13) (end 188.97 105.477) (width 0.2) (layer "B.Cu") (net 10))
 (segment (start 186.317 111.977) (end 186.317 108.13) (width 0.2) (layer "B.Cu") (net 10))
 (segment (start 188.97 105.477) (end 243.47 105.477) (width 0.2) (layer "B.Cu") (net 10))
 (segment (start 171.87 112.323) (end 185.971 112.323) (width 0.2) (layer "B.Cu") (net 10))
 (segment (start 185.971 112.323) (end 186.317 111.977) (width 0.2) (layer "B.Cu") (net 10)))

